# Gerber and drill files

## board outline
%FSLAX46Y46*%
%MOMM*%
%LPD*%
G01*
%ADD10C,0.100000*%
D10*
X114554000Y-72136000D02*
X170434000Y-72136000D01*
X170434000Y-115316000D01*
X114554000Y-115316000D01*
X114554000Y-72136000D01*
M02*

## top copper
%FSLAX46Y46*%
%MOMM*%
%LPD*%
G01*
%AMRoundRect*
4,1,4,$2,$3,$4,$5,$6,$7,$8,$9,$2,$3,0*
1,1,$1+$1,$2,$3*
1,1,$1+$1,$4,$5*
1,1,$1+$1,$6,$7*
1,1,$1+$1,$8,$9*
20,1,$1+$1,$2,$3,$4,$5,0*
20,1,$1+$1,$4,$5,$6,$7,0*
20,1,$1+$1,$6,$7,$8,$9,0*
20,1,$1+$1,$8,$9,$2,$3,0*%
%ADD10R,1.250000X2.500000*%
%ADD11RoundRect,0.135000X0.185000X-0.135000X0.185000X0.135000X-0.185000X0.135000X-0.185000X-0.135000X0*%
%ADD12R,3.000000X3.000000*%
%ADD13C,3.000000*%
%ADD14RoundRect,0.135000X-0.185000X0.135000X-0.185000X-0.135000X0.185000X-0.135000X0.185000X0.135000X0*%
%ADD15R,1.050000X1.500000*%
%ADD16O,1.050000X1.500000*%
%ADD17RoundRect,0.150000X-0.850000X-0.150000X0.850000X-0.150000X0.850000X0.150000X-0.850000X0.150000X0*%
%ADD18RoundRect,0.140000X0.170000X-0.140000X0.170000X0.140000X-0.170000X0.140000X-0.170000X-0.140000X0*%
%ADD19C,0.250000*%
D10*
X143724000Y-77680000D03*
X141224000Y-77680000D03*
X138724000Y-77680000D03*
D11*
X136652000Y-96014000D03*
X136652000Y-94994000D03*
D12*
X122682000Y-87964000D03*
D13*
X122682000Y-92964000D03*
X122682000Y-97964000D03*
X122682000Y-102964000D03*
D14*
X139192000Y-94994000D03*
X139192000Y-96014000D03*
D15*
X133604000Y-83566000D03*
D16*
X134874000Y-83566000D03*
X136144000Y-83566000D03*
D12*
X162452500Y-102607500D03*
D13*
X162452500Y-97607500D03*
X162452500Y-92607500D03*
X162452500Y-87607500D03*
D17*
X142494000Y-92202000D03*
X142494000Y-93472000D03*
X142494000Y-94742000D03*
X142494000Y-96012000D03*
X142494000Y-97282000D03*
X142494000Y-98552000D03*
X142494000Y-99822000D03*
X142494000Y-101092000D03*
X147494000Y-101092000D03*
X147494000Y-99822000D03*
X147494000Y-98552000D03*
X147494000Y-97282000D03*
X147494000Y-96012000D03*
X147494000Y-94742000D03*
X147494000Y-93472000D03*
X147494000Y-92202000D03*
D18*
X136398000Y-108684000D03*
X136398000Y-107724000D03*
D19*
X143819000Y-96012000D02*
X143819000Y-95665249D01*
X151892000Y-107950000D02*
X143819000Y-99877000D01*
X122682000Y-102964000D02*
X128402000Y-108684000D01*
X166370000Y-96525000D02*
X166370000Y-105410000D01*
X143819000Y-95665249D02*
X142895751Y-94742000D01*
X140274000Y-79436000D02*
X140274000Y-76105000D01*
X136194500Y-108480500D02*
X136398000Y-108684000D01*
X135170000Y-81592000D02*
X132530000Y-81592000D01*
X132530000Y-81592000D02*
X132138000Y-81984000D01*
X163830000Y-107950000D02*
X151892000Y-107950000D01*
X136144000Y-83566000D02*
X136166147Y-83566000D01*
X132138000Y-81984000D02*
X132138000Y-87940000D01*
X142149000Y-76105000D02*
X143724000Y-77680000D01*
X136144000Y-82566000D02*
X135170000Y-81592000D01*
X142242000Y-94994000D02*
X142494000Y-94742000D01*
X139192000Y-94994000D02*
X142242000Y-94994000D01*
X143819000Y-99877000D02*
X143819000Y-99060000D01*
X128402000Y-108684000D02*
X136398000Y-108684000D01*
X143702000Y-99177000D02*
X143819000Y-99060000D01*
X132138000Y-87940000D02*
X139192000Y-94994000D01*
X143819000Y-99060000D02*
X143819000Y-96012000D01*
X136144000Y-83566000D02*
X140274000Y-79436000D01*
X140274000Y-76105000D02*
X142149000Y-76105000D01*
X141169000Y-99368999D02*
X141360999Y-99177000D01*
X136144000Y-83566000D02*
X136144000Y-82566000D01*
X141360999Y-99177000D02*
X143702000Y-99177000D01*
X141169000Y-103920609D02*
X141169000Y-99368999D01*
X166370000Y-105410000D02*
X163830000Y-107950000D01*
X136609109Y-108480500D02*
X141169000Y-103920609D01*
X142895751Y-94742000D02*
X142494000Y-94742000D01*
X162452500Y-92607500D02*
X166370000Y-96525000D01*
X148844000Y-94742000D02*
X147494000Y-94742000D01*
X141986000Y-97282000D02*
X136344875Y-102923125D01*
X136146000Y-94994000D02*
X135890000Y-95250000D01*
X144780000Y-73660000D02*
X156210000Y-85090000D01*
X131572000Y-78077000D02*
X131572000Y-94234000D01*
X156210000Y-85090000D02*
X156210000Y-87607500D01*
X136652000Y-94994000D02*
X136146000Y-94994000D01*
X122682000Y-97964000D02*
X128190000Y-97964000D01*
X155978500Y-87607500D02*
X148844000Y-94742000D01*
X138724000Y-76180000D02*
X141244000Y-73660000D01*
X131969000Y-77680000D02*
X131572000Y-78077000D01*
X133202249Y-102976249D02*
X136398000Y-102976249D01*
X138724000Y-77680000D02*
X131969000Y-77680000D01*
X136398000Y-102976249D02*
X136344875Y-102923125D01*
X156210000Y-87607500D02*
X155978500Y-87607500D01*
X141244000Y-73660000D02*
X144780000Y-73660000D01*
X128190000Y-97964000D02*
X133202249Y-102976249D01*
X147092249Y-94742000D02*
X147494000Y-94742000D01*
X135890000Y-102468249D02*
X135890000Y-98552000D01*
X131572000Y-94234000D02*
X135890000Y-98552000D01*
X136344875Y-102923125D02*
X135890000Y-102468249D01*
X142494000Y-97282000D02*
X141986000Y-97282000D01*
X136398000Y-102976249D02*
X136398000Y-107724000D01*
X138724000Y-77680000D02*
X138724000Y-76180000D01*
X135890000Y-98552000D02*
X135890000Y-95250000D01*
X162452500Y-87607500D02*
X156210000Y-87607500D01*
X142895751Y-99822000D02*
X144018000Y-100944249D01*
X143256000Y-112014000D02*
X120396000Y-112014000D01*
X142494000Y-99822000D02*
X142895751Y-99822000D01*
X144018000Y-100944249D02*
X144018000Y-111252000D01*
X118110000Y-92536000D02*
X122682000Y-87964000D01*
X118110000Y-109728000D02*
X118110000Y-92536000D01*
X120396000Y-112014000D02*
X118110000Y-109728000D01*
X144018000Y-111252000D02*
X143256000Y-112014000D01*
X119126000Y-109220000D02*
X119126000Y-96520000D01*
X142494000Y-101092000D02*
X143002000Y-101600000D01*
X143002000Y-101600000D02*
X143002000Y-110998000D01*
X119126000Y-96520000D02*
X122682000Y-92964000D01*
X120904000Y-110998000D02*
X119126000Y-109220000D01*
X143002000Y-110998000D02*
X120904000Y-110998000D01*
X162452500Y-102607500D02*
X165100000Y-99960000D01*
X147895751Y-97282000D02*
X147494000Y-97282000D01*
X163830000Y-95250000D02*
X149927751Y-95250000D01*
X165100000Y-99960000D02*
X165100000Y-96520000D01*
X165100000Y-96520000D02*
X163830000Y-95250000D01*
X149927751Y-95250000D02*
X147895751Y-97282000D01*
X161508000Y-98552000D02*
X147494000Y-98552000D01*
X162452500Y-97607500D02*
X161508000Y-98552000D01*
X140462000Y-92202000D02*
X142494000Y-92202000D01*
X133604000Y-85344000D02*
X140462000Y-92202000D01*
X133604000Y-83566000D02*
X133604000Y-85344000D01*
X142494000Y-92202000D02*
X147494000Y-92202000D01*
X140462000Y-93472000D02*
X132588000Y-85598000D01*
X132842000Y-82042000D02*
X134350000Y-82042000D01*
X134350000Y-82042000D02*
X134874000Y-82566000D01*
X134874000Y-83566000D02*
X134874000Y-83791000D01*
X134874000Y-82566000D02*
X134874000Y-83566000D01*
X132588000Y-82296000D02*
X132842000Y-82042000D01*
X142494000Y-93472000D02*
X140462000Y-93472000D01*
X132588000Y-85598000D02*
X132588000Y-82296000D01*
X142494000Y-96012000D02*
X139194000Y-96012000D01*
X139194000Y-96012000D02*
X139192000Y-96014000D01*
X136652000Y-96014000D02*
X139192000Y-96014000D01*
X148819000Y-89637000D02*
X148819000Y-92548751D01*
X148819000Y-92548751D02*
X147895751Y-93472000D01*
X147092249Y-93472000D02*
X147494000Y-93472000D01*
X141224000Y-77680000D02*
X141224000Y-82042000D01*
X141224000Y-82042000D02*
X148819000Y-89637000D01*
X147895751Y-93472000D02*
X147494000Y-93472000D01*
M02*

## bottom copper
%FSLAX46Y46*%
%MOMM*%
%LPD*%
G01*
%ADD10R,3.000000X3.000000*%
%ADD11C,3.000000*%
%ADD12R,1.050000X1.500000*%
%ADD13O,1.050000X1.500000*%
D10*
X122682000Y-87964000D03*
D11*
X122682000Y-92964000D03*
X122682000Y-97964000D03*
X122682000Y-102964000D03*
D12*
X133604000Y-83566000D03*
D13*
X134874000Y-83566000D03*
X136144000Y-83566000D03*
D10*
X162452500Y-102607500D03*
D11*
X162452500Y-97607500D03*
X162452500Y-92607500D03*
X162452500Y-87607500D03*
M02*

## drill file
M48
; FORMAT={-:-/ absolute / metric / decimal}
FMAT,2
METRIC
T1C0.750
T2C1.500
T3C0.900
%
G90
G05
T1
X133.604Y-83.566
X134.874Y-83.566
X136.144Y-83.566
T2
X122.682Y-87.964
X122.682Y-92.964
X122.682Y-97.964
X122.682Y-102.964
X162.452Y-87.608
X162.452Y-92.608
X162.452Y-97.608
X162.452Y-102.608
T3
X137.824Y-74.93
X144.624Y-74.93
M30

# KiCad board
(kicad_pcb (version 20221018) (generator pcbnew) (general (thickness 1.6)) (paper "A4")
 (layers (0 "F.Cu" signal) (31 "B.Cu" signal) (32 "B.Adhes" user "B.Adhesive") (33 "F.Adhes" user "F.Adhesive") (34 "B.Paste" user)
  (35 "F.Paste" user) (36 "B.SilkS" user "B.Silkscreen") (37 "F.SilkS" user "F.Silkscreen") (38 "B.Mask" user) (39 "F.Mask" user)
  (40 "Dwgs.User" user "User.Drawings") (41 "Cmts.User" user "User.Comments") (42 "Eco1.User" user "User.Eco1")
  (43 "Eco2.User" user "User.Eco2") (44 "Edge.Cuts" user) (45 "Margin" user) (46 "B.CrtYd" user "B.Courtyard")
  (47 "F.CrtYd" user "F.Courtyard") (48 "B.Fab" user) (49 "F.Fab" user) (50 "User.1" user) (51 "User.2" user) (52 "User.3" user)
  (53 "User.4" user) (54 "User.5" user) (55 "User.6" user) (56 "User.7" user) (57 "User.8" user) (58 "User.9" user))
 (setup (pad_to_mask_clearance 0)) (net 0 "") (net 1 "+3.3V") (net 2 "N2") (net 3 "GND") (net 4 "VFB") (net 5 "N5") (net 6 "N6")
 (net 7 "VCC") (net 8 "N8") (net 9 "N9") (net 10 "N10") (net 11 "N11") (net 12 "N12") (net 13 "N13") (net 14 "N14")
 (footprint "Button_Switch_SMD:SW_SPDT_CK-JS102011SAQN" (layer "F.Cu") (at 141.224 74.93 180)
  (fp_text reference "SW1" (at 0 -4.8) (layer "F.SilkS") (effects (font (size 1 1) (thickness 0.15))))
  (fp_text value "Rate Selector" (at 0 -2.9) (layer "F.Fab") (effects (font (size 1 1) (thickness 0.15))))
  (pad "" np_thru_hole circle (at -3.4 0 180) (size 0.9 0.9) (drill 0.9) (layers "*.Cu" "*.Mask"))
  (pad "" np_thru_hole circle (at 3.4 0 180) (size 0.9 0.9) (drill 0.9) (layers "*.Cu" "*.Mask"))
  (pad "1" smd rect (at -2.5 -2.75 180) (size 1.25 2.5) (layers "F.Cu" "F.Paste" "F.Mask") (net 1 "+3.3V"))
  (pad "2" smd rect (at 0 -2.75 180) (size 1.25 2.5) (layers "F.Cu" "F.Paste" "F.Mask") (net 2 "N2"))
  (pad "3" smd rect (at 2.5 -2.75 180) (size 1.25 2.5) (layers "F.Cu" "F.Paste" "F.Mask") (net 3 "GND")))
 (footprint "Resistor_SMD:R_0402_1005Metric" (layer "F.Cu") (at 136.652 95.504 90)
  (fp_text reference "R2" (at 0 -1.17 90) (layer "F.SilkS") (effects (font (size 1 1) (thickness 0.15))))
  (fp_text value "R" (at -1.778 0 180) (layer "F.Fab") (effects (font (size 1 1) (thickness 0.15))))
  (pad "1" smd roundrect (at -0.51 0 90) (size 0.54 0.64) (layers "F.Cu" "F.Paste" "F.Mask") (roundrect_rratio 0.25) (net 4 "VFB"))
  (pad "2" smd roundrect (at 0.51 0 90) (size 0.54 0.64) (layers "F.Cu" "F.Paste" "F.Mask") (roundrect_rratio 0.25) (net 3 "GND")))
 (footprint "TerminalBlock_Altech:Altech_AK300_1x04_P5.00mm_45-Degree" (layer "F.Cu") (at 122.682 87.964 -90)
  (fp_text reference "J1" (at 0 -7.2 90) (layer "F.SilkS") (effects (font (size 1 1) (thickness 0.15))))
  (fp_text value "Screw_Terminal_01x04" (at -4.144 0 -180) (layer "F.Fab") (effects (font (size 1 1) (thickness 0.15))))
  (pad "1" thru_hole rect (at 0 0 270) (size 3 3) (drill 1.5) (layers "*.Cu" "*.Mask") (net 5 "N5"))
  (pad "2" thru_hole circle (at 5 0 270) (size 3 3) (drill 1.5) (layers "*.Cu" "*.Mask") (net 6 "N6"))
  (pad "3" thru_hole circle (at 10 0 270) (size 3 3) (drill 1.5) (layers "*.Cu" "*.Mask") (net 3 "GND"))
  (pad "4" thru_hole circle (at 15 0 270) (size 3 3) (drill 1.5) (layers "*.Cu" "*.Mask") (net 1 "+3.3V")))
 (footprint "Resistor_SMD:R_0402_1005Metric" (layer "F.Cu") (at 139.192 95.504 -90)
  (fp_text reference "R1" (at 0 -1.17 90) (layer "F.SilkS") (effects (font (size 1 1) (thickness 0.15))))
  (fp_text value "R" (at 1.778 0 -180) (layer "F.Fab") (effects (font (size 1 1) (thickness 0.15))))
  (pad "1" smd roundrect (at -0.51 0 270) (size 0.54 0.64) (layers "F.Cu" "F.Paste" "F.Mask") (roundrect_rratio 0.25) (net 1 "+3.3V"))
  (pad "2" smd roundrect (at 0.51 0 270) (size 0.54 0.64) (layers "F.Cu" "F.Paste" "F.Mask") (roundrect_rratio 0.25) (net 4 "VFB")))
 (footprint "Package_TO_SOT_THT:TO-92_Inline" (layer "F.Cu") (at 133.604 83.566)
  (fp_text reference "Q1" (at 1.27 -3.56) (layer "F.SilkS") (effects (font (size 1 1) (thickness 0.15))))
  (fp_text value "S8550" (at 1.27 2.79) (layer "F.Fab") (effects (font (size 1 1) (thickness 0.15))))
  (pad "1" thru_hole rect (at 0 0) (size 1.05 1.5) (drill 0.75) (layers "*.Cu" "*.Mask") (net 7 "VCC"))
  (pad "2" thru_hole oval (at 1.27 0) (size 1.05 1.5) (drill 0.75) (layers "*.Cu" "*.Mask") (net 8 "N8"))
  (pad "3" thru_hole oval (at 2.54 0) (size 1.05 1.5) (drill 0.75) (layers "*.Cu" "*.Mask") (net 1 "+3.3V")))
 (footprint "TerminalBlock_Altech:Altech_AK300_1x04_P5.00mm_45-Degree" (layer "F.Cu") (at 162.4525 102.6075 90)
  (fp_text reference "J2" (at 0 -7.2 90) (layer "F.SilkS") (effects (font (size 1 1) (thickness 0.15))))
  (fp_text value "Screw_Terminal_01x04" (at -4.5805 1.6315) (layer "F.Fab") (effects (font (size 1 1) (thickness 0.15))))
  (pad "1" thru_hole rect (at 0 0 90) (size 3 3) (drill 1.5) (layers "*.Cu" "*.Mask") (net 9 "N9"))
  (pad "2" thru_hole circle (at 5 0 90) (size 3 3) (drill 1.5) (layers "*.Cu" "*.Mask") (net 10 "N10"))
  (pad "3" thru_hole circle (at 10 0 90) (size 3 3) (drill 1.5) (layers "*.Cu" "*.Mask") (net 1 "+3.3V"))
  (pad "4" thru_hole circle (at 15 0 90) (size 3 3) (drill 1.5) (layers "*.Cu" "*.Mask") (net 3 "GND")))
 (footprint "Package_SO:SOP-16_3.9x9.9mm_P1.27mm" (layer "F.Cu") (at 144.994 96.647)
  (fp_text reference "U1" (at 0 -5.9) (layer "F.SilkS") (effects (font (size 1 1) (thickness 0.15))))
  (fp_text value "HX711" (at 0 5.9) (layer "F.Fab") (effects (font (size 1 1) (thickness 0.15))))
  (pad "1" smd roundrect (at -2.5 -4.445) (size 2 0.6) (layers "F.Cu" "F.Paste" "F.Mask") (roundrect_rratio 0.25) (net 7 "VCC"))
  (pad "2" smd roundrect (at -2.5 -3.175) (size 2 0.6) (layers "F.Cu" "F.Paste" "F.Mask") (roundrect_rratio 0.25) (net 8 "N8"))
  (pad "3" smd roundrect (at -2.5 -1.905) (size 2 0.6) (layers "F.Cu" "F.Paste" "F.Mask") (roundrect_rratio 0.25) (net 1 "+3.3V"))
  (pad "4" smd roundrect (at -2.5 -0.635) (size 2 0.6) (layers "F.Cu" "F.Paste" "F.Mask") (roundrect_rratio 0.25) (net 4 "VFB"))
  (pad "5" smd roundrect (at -2.5 0.635) (size 2 0.6) (layers "F.Cu" "F.Paste" "F.Mask") (roundrect_rratio 0.25) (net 3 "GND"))
  (pad "6" smd roundrect (at -2.5 1.905) (size 2 0.6) (layers "F.Cu" "F.Paste" "F.Mask") (roundrect_rratio 0.25) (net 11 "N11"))
  (pad "7" smd roundrect (at -2.5 3.175) (size 2 0.6) (layers "F.Cu" "F.Paste" "F.Mask") (roundrect_rratio 0.25) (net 5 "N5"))
  (pad "8" smd roundrect (at -2.5 4.445) (size 2 0.6) (layers "F.Cu" "F.Paste" "F.Mask") (roundrect_rratio 0.25) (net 6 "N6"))
  (pad "9" smd roundrect (at 2.5 4.445) (size 2 0.6) (layers "F.Cu" "F.Paste" "F.Mask") (roundrect_rratio 0.25) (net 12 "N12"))
  (pad "10" smd roundrect (at 2.5 3.175) (size 2 0.6) (layers "F.Cu" "F.Paste" "F.Mask") (roundrect_rratio 0.25) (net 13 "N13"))
  (pad "11" smd roundrect (at 2.5 1.905) (size 2 0.6) (layers "F.Cu" "F.Paste" "F.Mask") (roundrect_rratio 0.25) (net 10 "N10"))
  (pad "12" smd roundrect (at 2.5 0.635) (size 2 0.6) (layers "F.Cu" "F.Paste" "F.Mask") (roundrect_rratio 0.25) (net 9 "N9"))
  (pad "13" smd roundrect (at 2.5 -0.635) (size 2 0.6) (layers "F.Cu" "F.Paste" "F.Mask") (roundrect_rratio 0.25) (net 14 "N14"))
  (pad "14" smd roundrect (at 2.5 -1.905) (size 2 0.6) (layers "F.Cu" "F.Paste" "F.Mask") (roundrect_rratio 0.25) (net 3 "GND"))
  (pad "15" smd roundrect (at 2.5 -3.175) (size 2 0.6) (layers "F.Cu" "F.Paste" "F.Mask") (roundrect_rratio 0.25) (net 2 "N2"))
  (pad "16" smd roundrect (at 2.5 -4.445) (size 2 0.6) (layers "F.Cu" "F.Paste" "F.Mask") (roundrect_rratio 0.25) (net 7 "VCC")))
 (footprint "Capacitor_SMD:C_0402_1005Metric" (layer "F.Cu") (at 136.398 108.204 90)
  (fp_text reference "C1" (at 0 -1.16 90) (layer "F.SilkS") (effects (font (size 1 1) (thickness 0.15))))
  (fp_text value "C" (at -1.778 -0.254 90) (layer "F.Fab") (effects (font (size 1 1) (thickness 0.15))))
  (pad "1" smd roundrect (at -0.48 0 90) (size 0.56 0.62) (layers "F.Cu" "F.Paste" "F.Mask") (roundrect_rratio 0.25) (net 1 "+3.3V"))
  (pad "2" smd roundrect (at 0.48 0 90) (size 0.56 0.62) (layers "F.Cu" "F.Paste" "F.Mask") (roundrect_rratio 0.25) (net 3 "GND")))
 (gr_rect (start 114.554 72.136) (end 170.434 115.316) (stroke (width 0.1) (type default)) (fill none) (layer "Edge.Cuts"))
 (segment (start 143.819 96.012) (end 143.819 95.665249) (width 0.25) (layer "F.Cu") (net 1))
 (segment (start 151.892 107.95) (end 143.819 99.877) (width 0.25) (layer "F.Cu") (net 1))
 (segment (start 122.682 102.964) (end 128.402 108.684) (width 0.25) (layer "F.Cu") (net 1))
 (segment (start 166.37 96.525) (end 166.37 105.41) (width 0.25) (layer "F.Cu") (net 1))
 (segment (start 143.819 95.665249) (end 142.895751 94.742) (width 0.25) (layer "F.Cu") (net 1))
 (segment (start 140.274 79.436) (end 140.274 76.105) (width 0.25) (layer "F.Cu") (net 1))
 (segment (start 136.1945 108.4805) (end 136.398 108.684) (width 0.25) (layer "F.Cu") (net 1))
 (segment (start 135.17 81.592) (end 132.53 81.592) (width 0.25) (layer "F.Cu") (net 1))
 (segment (start 132.53 81.592) (end 132.138 81.984) (width 0.25) (layer "F.Cu") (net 1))
 (segment (start 163.83 107.95) (end 151.892 107.95) (width 0.25) (layer "F.Cu") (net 1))
 (segment (start 136.144 83.566) (end 136.166147 83.566) (width 0.25) (layer "F.Cu") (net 1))
 (segment (start 132.138 81.984) (end 132.138 87.94) (width 0.25) (layer "F.Cu") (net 1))
 (segment (start 142.149 76.105) (end 143.724 77.68) (width 0.25) (layer "F.Cu") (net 1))
 (segment (start 136.144 82.566) (end 135.17 81.592) (width 0.25) (layer "F.Cu") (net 1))
 (segment (start 142.242 94.994) (end 142.494 94.742) (width 0.25) (layer "F.Cu") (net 1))
 (segment (start 139.192 94.994) (end 142.242 94.994) (width 0.25) (layer "F.Cu") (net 1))
 (segment (start 143.819 99.877) (end 143.819 99.06) (width 0.25) (layer "F.Cu") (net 1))
 (segment (start 128.402 108.684) (end 136.398 108.684) (width 0.25) (layer "F.Cu") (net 1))
 (segment (start 143.702 99.177) (end 143.819 99.06) (width 0.25) (layer "F.Cu") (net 1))
 (segment (start 132.138 87.94) (end 139.192 94.994) (width 0.25) (layer "F.Cu") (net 1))
 (segment (start 143.819 99.06) (end 143.819 96.012) (width 0.25) (layer "F.Cu") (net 1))
 (segment (start 136.144 83.566) (end 140.274 79.436) (width 0.25) (layer "F.Cu") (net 1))
 (segment (start 140.274 76.105) (end 142.149 76.105) (width 0.25) (layer "F.Cu") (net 1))
 (segment (start 141.169 99.368999) (end 141.360999 99.177) (width 0.25) (layer "F.Cu") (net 1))
 (segment (start 136.144 83.566) (end 136.144 82.566) (width 0.25) (layer "F.Cu") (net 1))
 (segment (start 141.360999 99.177) (end 143.702 99.177) (width 0.25) (layer "F.Cu") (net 1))
 (segment (start 141.169 103.920609) (end 141.169 99.368999) (width 0.25) (layer "F.Cu") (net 1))
 (segment (start 166.37 105.41) (end 163.83 107.95) (width 0.25) (layer "F.Cu") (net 1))
 (segment (start 136.609109 108.4805) (end 141.169 103.920609) (width 0.25) (layer "F.Cu") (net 1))
 (segment (start 142.895751 94.742) (end 142.494 94.742) (width 0.25) (layer "F.Cu") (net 1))
 (segment (start 162.4525 92.6075) (end 166.37 96.525) (width 0.25) (layer "F.Cu") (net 1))
 (segment (start 148.844 94.742) (end 147.494 94.742) (width 0.25) (layer "F.Cu") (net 3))
 (segment (start 141.986 97.282) (end 136.344875 102.923125) (width 0.25) (layer "F.Cu") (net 3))
 (segment (start 136.146 94.994) (end 135.89 95.25) (width 0.25) (layer "F.Cu") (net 3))
 (segment (start 144.78 73.66) (end 156.21 85.09) (width 0.25) (layer "F.Cu") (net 3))
 (segment (start 131.572 78.077) (end 131.572 94.234) (width 0.25) (layer "F.Cu") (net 3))
 (segment (start 156.21 85.09) (end 156.21 87.6075) (width 0.25) (layer "F.Cu") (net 3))
 (segment (start 136.652 94.994) (end 136.146 94.994) (width 0.25) (layer "F.Cu") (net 3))
 (segment (start 122.682 97.964) (end 128.19 97.964) (width 0.25) (layer "F.Cu") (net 3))
 (segment (start 155.9785 87.6075) (end 148.844 94.742) (width 0.25) (layer "F.Cu") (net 3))
 (segment (start 138.724 76.18) (end 141.244 73.66) (width 0.25) (layer "F.Cu") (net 3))
 (segment (start 131.969 77.68) (end 131.572 78.077) (width 0.25) (layer "F.Cu") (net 3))
 (segment (start 133.202249 102.976249) (end 136.398 102.976249) (width 0.25) (layer "F.Cu") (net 3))
 (segment (start 138.724 77.68) (end 131.969 77.68) (width 0.25) (layer "F.Cu") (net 3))
 (segment (start 136.398 102.976249) (end 136.344875 102.923125) (width 0.25) (layer "F.Cu") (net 3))
 (segment (start 156.21 87.6075) (end 155.9785 87.6075) (width 0.25) (layer "F.Cu") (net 3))
 (segment (start 141.244 73.66) (end 144.78 73.66) (width 0.25) (layer "F.Cu") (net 3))
 (segment (start 128.19 97.964) (end 133.202249 102.976249) (width 0.25) (layer "F.Cu") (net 3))
 (segment (start 147.092249 94.742) (end 147.494 94.742) (width 0.25) (layer "F.Cu") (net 3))
 (segment (start 135.89 102.468249) (end 135.89 98.552) (width 0.25) (layer "F.Cu") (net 3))
 (segment (start 131.572 94.234) (end 135.89 98.552) (width 0.25) (layer "F.Cu") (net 3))
 (segment (start 136.344875 102.923125) (end 135.89 102.468249) (width 0.25) (layer "F.Cu") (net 3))
 (segment (start 142.494 97.282) (end 141.986 97.282) (width 0.25) (layer "F.Cu") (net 3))
 (segment (start 136.398 102.976249) (end 136.398 107.724) (width 0.25) (layer "F.Cu") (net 3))
 (segment (start 138.724 77.68) (end 138.724 76.18) (width 0.25) (layer "F.Cu") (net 3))
 (segment (start 135.89 98.552) (end 135.89 95.25) (width 0.25) (layer "F.Cu") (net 3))
 (segment (start 162.4525 87.6075) (end 156.21 87.6075) (width 0.25) (layer "F.Cu") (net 3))
 (segment (start 142.895751 99.822) (end 144.018 100.944249) (width 0.25) (layer "F.Cu") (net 5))
 (segment (start 143.256 112.014) (end 120.396 112.014) (width 0.25) (layer "F.Cu") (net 5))
 (segment (start 142.494 99.822) (end 142.895751 99.822) (width 0.25) (layer "F.Cu") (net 5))
 (segment (start 144.018 100.944249) (end 144.018 111.252) (width 0.25) (layer "F.Cu") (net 5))
 (segment (start 118.11 92.536) (end 122.682 87.964) (width 0.25) (layer "F.Cu") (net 5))
 (segment (start 118.11 109.728) (end 118.11 92.536) (width 0.25) (layer "F.Cu") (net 5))
 (segment (start 120.396 112.014) (end 118.11 109.728) (width 0.25) (layer "F.Cu") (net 5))
 (segment (start 144.018 111.252) (end 143.256 112.014) (width 0.25) (layer "F.Cu") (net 5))
 (segment (start 119.126 109.22) (end 119.126 96.52) (width 0.25) (layer "F.Cu") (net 6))
 (segment (start 142.494 101.092) (end 143.002 101.6) (width 0.25) (layer "F.Cu") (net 6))
 (segment (start 143.002 101.6) (end 143.002 110.998) (width 0.25) (layer "F.Cu") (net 6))
 (segment (start 119.126 96.52) (end 122.682 92.964) (width 0.25) (layer "F.Cu") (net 6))
 (segment (start 120.904 110.998) (end 119.126 109.22) (width 0.25) (layer "F.Cu") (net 6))
 (segment (start 143.002 110.998) (end 120.904 110.998) (width 0.25) (layer "F.Cu") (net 6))
 (segment (start 162.4525 102.6075) (end 165.1 99.96) (width 0.25) (layer "F.Cu") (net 9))
 (segment (start 147.895751 97.282) (end 147.494 97.282) (width 0.25) (layer "F.Cu") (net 9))
 (segment (start 163.83 95.25) (end 149.927751 95.25) (width 0.25) (layer "F.Cu") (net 9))
 (segment (start 165.1 99.96) (end 165.1 96.52) (width 0.25) (layer "F.Cu") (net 9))
 (segment (start 165.1 96.52) (end 163.83 95.25) (width 0.25) (layer "F.Cu") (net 9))
 (segment (start 149.927751 95.25) (end 147.895751 97.282) (width 0.25) (layer "F.Cu") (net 9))
 (segment (start 161.508 98.552) (end 147.494 98.552) (width 0.25) (layer "F.Cu") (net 10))
 (segment (start 162.4525 97.6075) (end 161.508 98.552) (width 0.25) (layer "F.Cu") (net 10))
 (segment (start 140.462 92.202) (end 142.494 92.202) (width 0.25) (layer "F.Cu") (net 7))
 (segment (start 133.604 85.344) (end 140.462 92.202) (width 0.25) (layer "F.Cu") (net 7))
 (segment (start 133.604 83.566) (end 133.604 85.344) (width 0.25) (layer "F.Cu") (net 7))
 (segment (start 142.494 92.202) (end 147.494 92.202) (width 0.25) (layer "F.Cu") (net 7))
 (segment (start 140.462 93.472) (end 132.588 85.598) (width 0.25) (layer "F.Cu") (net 8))
 (segment (start 132.842 82.042) (end 134.35 82.042) (width 0.25) (layer "F.Cu") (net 8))
 (segment (start 134.35 82.042) (end 134.874 82.566) (width 0.25) (layer "F.Cu") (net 8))
 (segment (start 134.874 83.566) (end 134.874 83.791) (width 0.25) (layer "F.Cu") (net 8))
 (segment (start 134.874 82.566) (end 134.874 83.566) (width 0.25) (layer "F.Cu") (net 8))
 (segment (start 132.588 82.296) (end 132.842 82.042) (width 0.25) (layer "F.Cu") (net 8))
 (segment (start 142.494 93.472) (end 140.462 93.472) (width 0.25) (layer "F.Cu") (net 8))
 (segment (start 132.588 85.598) (end 132.588 82.296) (width 0.25) (layer "F.Cu") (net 8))
 (segment (start 142.494 96.012) (end 139.194 96.012) (width 0.25) (layer "F.Cu") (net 4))
 (segment (start 139.194 96.012) (end 139.192 96.014) (width 0.25) (layer "F.Cu") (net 4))
 (segment (start 136.652 96.014) (end 139.192 96.014) (width 0.25) (layer "F.Cu") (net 4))
 (segment (start 148.819 89.637) (end 148.819 92.548751) (width 0.25) (layer "F.Cu") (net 2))
 (segment (start 148.819 92.548751) (end 147.895751 93.472) (width 0.25) (layer "F.Cu") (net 2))
 (segment (start 147.092249 93.472) (end 147.494 93.472) (width 0.25) (layer "F.Cu") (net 2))
 (segment (start 141.224 77.68) (end 141.224 82.042) (width 0.25) (layer "F.Cu") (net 2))
 (segment (start 141.224 82.042) (end 148.819 89.637) (width 0.25) (layer "F.Cu") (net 2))
 (segment (start 147.895751 93.472) (end 147.494 93.472) (width 0.25) (layer "F.Cu") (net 2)))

